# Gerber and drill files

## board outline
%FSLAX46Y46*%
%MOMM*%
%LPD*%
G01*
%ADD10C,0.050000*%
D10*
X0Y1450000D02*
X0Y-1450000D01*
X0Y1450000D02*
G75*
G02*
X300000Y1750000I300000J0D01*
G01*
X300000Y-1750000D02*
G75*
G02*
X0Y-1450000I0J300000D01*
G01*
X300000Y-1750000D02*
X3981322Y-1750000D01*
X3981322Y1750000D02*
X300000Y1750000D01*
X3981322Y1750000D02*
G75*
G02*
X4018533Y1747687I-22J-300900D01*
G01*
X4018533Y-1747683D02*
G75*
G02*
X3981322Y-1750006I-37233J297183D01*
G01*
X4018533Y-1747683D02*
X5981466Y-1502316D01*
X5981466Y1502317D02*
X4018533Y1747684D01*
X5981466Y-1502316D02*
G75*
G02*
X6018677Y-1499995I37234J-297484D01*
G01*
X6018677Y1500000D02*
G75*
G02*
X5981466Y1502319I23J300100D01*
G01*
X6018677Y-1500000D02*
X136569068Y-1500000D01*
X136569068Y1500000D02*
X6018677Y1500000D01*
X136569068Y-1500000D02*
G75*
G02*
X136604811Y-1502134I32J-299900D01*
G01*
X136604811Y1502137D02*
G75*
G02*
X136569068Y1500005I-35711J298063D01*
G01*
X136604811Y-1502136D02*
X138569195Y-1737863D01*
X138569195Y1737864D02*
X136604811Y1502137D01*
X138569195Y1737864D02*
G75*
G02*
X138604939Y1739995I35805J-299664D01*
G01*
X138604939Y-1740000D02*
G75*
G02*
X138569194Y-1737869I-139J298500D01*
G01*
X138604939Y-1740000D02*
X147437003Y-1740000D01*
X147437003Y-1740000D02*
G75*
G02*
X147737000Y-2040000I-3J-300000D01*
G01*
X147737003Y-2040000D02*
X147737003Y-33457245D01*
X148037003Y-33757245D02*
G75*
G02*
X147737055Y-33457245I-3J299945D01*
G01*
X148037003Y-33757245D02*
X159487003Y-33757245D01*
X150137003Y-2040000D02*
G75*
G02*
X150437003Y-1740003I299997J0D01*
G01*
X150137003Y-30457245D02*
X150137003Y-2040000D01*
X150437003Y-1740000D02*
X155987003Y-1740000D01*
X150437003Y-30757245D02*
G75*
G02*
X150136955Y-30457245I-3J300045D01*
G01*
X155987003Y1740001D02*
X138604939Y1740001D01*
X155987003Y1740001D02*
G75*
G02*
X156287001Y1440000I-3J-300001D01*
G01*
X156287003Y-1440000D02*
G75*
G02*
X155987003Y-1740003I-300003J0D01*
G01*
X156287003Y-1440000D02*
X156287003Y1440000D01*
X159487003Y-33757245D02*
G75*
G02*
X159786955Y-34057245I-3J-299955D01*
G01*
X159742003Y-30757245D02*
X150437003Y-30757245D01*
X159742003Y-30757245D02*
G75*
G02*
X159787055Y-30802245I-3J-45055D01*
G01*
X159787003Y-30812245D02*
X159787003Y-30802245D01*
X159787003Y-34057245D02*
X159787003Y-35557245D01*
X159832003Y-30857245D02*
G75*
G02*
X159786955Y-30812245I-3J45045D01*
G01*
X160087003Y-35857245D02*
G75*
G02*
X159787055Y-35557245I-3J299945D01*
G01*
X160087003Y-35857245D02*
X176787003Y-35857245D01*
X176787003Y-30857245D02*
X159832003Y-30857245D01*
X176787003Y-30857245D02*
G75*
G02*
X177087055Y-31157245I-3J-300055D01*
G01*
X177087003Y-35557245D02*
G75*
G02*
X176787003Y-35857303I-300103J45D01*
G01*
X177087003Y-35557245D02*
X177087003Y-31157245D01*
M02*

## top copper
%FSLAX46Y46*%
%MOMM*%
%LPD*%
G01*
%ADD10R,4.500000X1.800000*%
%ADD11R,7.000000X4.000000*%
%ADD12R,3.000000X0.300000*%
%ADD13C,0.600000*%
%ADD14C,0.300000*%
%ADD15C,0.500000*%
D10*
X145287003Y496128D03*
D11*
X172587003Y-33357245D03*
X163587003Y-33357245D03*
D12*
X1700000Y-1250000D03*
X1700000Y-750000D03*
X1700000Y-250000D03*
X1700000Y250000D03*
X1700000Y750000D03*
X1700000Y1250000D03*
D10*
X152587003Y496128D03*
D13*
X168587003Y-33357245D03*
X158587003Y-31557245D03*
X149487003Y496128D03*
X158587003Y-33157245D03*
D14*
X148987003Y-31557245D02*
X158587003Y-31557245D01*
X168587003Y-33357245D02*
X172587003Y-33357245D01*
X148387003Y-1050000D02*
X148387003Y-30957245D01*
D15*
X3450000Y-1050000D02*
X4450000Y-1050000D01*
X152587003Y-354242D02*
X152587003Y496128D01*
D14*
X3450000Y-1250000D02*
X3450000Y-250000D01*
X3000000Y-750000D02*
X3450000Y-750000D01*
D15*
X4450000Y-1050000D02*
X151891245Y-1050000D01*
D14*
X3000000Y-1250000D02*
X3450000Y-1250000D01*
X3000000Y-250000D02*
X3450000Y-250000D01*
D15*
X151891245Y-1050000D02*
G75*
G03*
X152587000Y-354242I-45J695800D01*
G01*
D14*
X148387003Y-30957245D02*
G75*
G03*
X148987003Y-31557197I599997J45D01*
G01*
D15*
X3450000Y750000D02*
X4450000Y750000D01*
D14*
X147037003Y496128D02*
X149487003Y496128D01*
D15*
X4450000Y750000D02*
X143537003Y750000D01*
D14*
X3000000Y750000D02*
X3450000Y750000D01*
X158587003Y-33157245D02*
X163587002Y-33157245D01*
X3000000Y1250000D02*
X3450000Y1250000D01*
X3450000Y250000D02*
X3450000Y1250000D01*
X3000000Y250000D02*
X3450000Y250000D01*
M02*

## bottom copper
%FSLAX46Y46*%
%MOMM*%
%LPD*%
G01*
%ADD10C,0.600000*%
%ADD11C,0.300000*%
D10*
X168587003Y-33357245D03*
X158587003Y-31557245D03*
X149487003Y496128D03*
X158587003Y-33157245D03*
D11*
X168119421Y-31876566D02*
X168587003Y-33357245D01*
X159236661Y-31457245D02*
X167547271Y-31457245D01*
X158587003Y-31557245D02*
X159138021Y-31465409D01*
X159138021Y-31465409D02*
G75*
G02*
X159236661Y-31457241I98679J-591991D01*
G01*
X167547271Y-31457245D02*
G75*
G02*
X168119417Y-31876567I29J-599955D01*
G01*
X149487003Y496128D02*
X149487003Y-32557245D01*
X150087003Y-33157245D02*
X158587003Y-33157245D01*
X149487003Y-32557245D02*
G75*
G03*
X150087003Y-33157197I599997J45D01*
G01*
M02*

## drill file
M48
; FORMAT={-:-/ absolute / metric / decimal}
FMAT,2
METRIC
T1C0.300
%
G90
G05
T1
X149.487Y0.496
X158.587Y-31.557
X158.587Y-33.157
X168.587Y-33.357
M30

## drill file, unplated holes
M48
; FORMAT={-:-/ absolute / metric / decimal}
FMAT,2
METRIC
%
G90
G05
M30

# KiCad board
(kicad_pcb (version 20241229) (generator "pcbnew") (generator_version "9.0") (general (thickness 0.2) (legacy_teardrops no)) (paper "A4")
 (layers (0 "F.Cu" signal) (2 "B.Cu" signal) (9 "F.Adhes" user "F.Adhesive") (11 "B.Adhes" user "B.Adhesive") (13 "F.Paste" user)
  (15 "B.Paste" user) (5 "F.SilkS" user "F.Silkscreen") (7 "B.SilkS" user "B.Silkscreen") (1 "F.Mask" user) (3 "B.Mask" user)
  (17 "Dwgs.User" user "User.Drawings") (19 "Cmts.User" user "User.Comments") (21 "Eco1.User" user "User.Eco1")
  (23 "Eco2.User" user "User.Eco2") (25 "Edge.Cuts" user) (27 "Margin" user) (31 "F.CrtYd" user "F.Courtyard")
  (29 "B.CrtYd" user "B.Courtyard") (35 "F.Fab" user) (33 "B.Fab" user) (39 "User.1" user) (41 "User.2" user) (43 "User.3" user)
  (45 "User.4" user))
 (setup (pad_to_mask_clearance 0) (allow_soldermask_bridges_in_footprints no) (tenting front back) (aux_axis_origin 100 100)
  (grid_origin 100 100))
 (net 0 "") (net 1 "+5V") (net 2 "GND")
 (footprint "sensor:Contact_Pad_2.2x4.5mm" (layer "F.Cu") (at 245.287003 99.503872)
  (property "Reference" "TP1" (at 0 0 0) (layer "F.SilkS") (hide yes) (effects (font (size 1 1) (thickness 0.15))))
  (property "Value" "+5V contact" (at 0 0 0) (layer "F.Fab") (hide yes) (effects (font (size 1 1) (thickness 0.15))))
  (pad "1" smd rect (at 0 0) (size 4.5 1.8) (layers "F.Cu" "F.Mask") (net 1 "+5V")))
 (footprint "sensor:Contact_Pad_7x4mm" (layer "F.Cu") (at 272.587003 133.357245)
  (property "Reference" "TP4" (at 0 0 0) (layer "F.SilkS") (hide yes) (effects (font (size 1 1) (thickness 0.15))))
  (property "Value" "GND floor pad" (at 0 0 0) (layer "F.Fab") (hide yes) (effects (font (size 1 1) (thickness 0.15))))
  (pad "1" smd rect (at 0 0) (size 7 4) (layers "F.Cu" "F.Mask") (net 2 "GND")))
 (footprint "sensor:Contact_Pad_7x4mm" (layer "F.Cu") (at 263.587003 133.357245)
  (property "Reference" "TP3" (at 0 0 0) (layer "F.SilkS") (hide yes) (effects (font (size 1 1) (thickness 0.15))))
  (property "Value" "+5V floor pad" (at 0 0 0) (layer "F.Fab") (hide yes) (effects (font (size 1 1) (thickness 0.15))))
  (pad "1" smd rect (at 0 0) (size 7 4) (layers "F.Cu" "F.Mask") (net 1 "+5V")))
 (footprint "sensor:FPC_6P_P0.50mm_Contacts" (layer "F.Cu") (at 101.7 100)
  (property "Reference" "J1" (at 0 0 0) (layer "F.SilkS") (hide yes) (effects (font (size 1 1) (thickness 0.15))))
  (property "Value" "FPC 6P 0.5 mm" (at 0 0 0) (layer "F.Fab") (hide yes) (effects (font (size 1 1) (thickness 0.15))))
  (pad "1" smd rect (at 0 1.25) (size 3 0.3) (layers "F.Cu" "F.Mask") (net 2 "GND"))
  (pad "2" smd rect (at 0 0.75) (size 3 0.3) (layers "F.Cu" "F.Mask") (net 2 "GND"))
  (pad "3" smd rect (at 0 0.25) (size 3 0.3) (layers "F.Cu" "F.Mask") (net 2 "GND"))
  (pad "4" smd rect (at 0 -0.25) (size 3 0.3) (layers "F.Cu" "F.Mask") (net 1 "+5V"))
  (pad "5" smd rect (at 0 -0.75) (size 3 0.3) (layers "F.Cu" "F.Mask") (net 1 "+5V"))
  (pad "6" smd rect (at 0 -1.25) (size 3 0.3) (layers "F.Cu" "F.Mask") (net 1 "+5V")))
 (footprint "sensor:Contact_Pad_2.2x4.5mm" (layer "F.Cu") (at 252.587003 99.503872)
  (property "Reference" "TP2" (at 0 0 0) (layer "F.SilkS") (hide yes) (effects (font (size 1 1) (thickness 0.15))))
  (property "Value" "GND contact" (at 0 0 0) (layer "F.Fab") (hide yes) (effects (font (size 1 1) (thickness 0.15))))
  (pad "1" smd rect (at 0 0) (size 4.5 1.8) (layers "F.Cu" "F.Mask") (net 2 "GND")))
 (gr_line (start 100 98.55) (end 100 101.45) (stroke (width 0.05) (type default)) (layer "Edge.Cuts"))
 (gr_arc (start 100 98.55) (mid 100.087868 98.337868) (end 100.3 98.25) (stroke (width 0.05) (type default)) (layer "Edge.Cuts"))
 (gr_arc (start 100.3 101.75) (mid 100.087868 101.662132) (end 100 101.45) (stroke (width 0.05) (type default)) (layer "Edge.Cuts"))
 (gr_line (start 100.3 101.75) (end 103.981322 101.75) (stroke (width 0.05) (type default)) (layer "Edge.Cuts"))
 (gr_line (start 103.981322 98.25) (end 100.3 98.25) (stroke (width 0.05) (type default)) (layer "Edge.Cuts"))
 (gr_arc (start 103.981322 98.25) (mid 103.999963 98.250581) (end 104.018533 98.252316) (stroke (width 0.05) (type default))
  (layer "Edge.Cuts"))
 (gr_arc (start 104.018533 101.747683) (mid 103.999964 101.749421) (end 103.981322 101.75) (stroke (width 0.05) (type default))
  (layer "Edge.Cuts"))
 (gr_line (start 104.018533 101.747683) (end 105.981466 101.502316) (stroke (width 0.05) (type default)) (layer "Edge.Cuts"))
 (gr_line (start 105.981466 98.497683) (end 104.018533 98.252316) (stroke (width 0.05) (type default)) (layer "Edge.Cuts"))
 (gr_arc (start 105.981466 101.502316) (mid 106.000036 101.500579) (end 106.018677 101.5) (stroke (width 0.05) (type default))
  (layer "Edge.Cuts"))
 (gr_arc (start 106.018677 98.5) (mid 106.000036 98.49942) (end 105.981466 98.497683) (stroke (width 0.05) (type default))
  (layer "Edge.Cuts"))
 (gr_line (start 106.018677 101.5) (end 236.569068 101.5) (stroke (width 0.05) (type default)) (layer "Edge.Cuts"))
 (gr_line (start 236.569068 98.5) (end 106.018677 98.5) (stroke (width 0.05) (type default)) (layer "Edge.Cuts"))
 (gr_arc (start 236.569068 101.5) (mid 236.586971 101.500534) (end 236.604811 101.502136) (stroke (width 0.05) (type default))
  (layer "Edge.Cuts"))
 (gr_arc (start 236.604811 98.497863) (mid 236.586971 98.499465) (end 236.569068 98.5) (stroke (width 0.05) (type default))
  (layer "Edge.Cuts"))
 (gr_line (start 236.604811 101.502136) (end 238.569195 101.737863) (stroke (width 0.05) (type default)) (layer "Edge.Cuts"))
 (gr_line (start 238.569195 98.262136) (end 236.604811 98.497863) (stroke (width 0.05) (type default)) (layer "Edge.Cuts"))
 (gr_arc (start 238.569195 98.262136) (mid 238.587035 98.260537) (end 238.604939 98.259999) (stroke (width 0.05) (type default))
  (layer "Edge.Cuts"))
 (gr_arc (start 238.604939 101.74) (mid 238.587035 101.739468) (end 238.569195 101.737863) (stroke (width 0.05) (type default))
  (layer "Edge.Cuts"))
 (gr_line (start 238.604939 101.74) (end 247.437003 101.74) (stroke (width 0.05) (type default)) (layer "Edge.Cuts"))
 (gr_arc (start 247.437003 101.74) (mid 247.649135 101.827867) (end 247.737003 102.04) (stroke (width 0.05) (type default))
  (layer "Edge.Cuts"))
 (gr_line (start 247.737003 102.04) (end 247.737003 133.457245) (stroke (width 0.05) (type default)) (layer "Edge.Cuts"))
 (gr_arc (start 248.037003 133.757245) (mid 247.824853 133.669381) (end 247.737003 133.457245) (stroke (width 0.05) (type default))
  (layer "Edge.Cuts"))
 (gr_line (start 248.037003 133.757245) (end 259.487003 133.757245) (stroke (width 0.05) (type default)) (layer "Edge.Cuts"))
 (gr_arc (start 250.137003 102.04) (mid 250.224871 101.827867) (end 250.437003 101.74) (stroke (width 0.05) (type default))
  (layer "Edge.Cuts"))
 (gr_line (start 250.137003 130.457245) (end 250.137003 102.04) (stroke (width 0.05) (type default)) (layer "Edge.Cuts"))
 (gr_line (start 250.437003 101.74) (end 255.987003 101.74) (stroke (width 0.05) (type default)) (layer "Edge.Cuts"))
 (gr_arc (start 250.437003 130.757245) (mid 250.224871 130.669377) (end 250.137003 130.457245) (stroke (width 0.05) (type default))
  (layer "Edge.Cuts"))
 (gr_line (start 255.987003 98.259999) (end 238.604939 98.259999) (stroke (width 0.05) (type default)) (layer "Edge.Cuts"))
 (gr_arc (start 255.987003 98.259999) (mid 256.199134 98.347868) (end 256.287003 98.56) (stroke (width 0.05) (type default))
  (layer "Edge.Cuts"))
 (gr_arc (start 256.287003 101.44) (mid 256.199135 101.652133) (end 255.987003 101.74) (stroke (width 0.05) (type default))
  (layer "Edge.Cuts"))
 (gr_line (start 256.287003 101.44) (end 256.287003 98.56) (stroke (width 0.05) (type default)) (layer "Edge.Cuts"))
 (gr_arc (start 259.487003 133.757245) (mid 259.699135 133.845113) (end 259.787003 134.057245) (stroke (width 0.05) (type default))
  (layer "Edge.Cuts"))
 (gr_line (start 259.742003 130.757245) (end 250.437003 130.757245) (stroke (width 0.05) (type default)) (layer "Edge.Cuts"))
 (gr_arc (start 259.742003 130.757245) (mid 259.773805 130.770429) (end 259.787003 130.802245) (stroke (width 0.05) (type default))
  (layer "Edge.Cuts"))
 (gr_line (start 259.787003 130.812245) (end 259.787003 130.802245) (stroke (width 0.05) (type default)) (layer "Edge.Cuts"))
 (gr_line (start 259.787003 134.057245) (end 259.787003 135.557245) (stroke (width 0.05) (type default)) (layer "Edge.Cuts"))
 (gr_arc (start 259.832003 130.857245) (mid 259.800184 130.844065) (end 259.787003 130.812245) (stroke (width 0.05) (type default))
  (layer "Edge.Cuts"))
 (gr_arc (start 260.087003 135.857245) (mid 259.874853 135.769381) (end 259.787003 135.557245) (stroke (width 0.05) (type default))
  (layer "Edge.Cuts"))
 (gr_line (start 260.087003 135.857245) (end 276.787003 135.857245) (stroke (width 0.05) (type default)) (layer "Edge.Cuts"))
 (gr_line (start 276.787003 130.857245) (end 259.832003 130.857245) (stroke (width 0.05) (type default)) (layer "Edge.Cuts"))
 (gr_arc (start 276.787003 130.857245) (mid 276.999117 130.945117) (end 277.087003 131.157245) (stroke (width 0.05) (type default))
  (layer "Edge.Cuts"))
 (gr_arc (start 277.087003 135.557245) (mid 276.999119 135.769349) (end 276.787003 135.857245) (stroke (width 0.05) (type default))
  (layer "Edge.Cuts"))
 (gr_line (start 277.087003 135.557245) (end 277.087003 131.157245) (stroke (width 0.05) (type default)) (layer "Edge.Cuts"))
 (segment (start 248.987003 131.557245) (end 258.587003 131.557245) (width 0.3) (layer "F.Cu") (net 2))
 (segment (start 268.587003 133.357245) (end 272.587003 133.357245) (width 0.3) (layer "F.Cu") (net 2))
 (segment (start 248.387003 101.05) (end 248.387003 130.957245) (width 0.3) (layer "F.Cu") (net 2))
 (segment (start 103.45 101.05) (end 104.45 101.05) (width 0.5) (layer "F.Cu") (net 2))
 (segment (start 252.587003 100.354242) (end 252.587003 99.503872) (width 0.5) (layer "F.Cu") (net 2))
 (segment (start 103.45 101.25) (end 103.45 100.25) (width 0.3) (layer "F.Cu") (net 2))
 (segment (start 103 100.75) (end 103.45 100.75) (width 0.3) (layer "F.Cu") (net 2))
 (segment (start 104.45 101.05) (end 251.891245 101.05) (width 0.5) (layer "F.Cu") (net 2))
 (segment (start 103 101.25) (end 103.45 101.25) (width 0.3) (layer "F.Cu") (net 2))
 (segment (start 103 100.25) (end 103.45 100.25) (width 0.3) (layer "F.Cu") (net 2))
 (via (at 268.587003 133.357245) (size 0.6) (drill 0.3) (layers "F.Cu" "B.Cu") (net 2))
 (via (at 258.587003 131.557245) (size 0.6) (drill 0.3) (layers "F.Cu" "B.Cu") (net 2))
 (arc (start 251.891245 101.05) (mid 252.38322 100.846217) (end 252.587003 100.354242) (width 0.5) (layer "F.Cu") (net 2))
 (arc (start 248.387003 130.957245) (mid 248.562739 131.381509) (end 248.987003 131.557245) (width 0.3) (layer "F.Cu") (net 2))
 (segment (start 268.119421 131.876566) (end 268.587003 133.357245) (width 0.3) (layer "B.Cu") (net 2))
 (segment (start 259.236661 131.457245) (end 267.547271 131.457245) (width 0.3) (layer "B.Cu") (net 2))
 (segment (start 258.587003 131.557245) (end 259.138021 131.465409) (width 0.3) (layer "B.Cu") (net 2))
 (arc (start 259.138021 131.465409) (mid 259.187173 131.45929) (end 259.236661 131.457245) (width 0.3) (layer "B.Cu") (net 2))
 (arc (start 267.547271 131.457245) (mid 267.901949 131.573299) (end 268.119421 131.876566) (width 0.3) (layer "B.Cu") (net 2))
 (segment (start 103.45 99.25) (end 104.45 99.25) (width 0.5) (layer "F.Cu") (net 1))
 (segment (start 247.037003 99.503872) (end 249.487003 99.503872) (width 0.3) (layer "F.Cu") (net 1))
 (segment (start 104.45 99.25) (end 243.537003 99.25) (width 0.5) (layer "F.Cu") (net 1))
 (segment (start 103 99.25) (end 103.45 99.25) (width 0.3) (layer "F.Cu") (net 1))
 (segment (start 258.587003 133.157245) (end 263.587002 133.157245) (width 0.3) (layer "F.Cu") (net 1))
 (segment (start 103 98.75) (end 103.45 98.75) (width 0.3) (layer "F.Cu") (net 1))
 (segment (start 103.45 99.75) (end 103.45 98.75) (width 0.3) (layer "F.Cu") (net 1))
 (segment (start 103 99.75) (end 103.45 99.75) (width 0.3) (layer "F.Cu") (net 1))
 (via (at 249.487003 99.503872) (size 0.6) (drill 0.3) (layers "F.Cu" "B.Cu") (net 1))
 (via (at 258.587003 133.157245) (size 0.6) (drill 0.3) (layers "F.Cu" "B.Cu") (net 1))
 (segment (start 249.487003 99.503872) (end 249.487003 132.557245) (width 0.3) (layer "B.Cu") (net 1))
 (segment (start 250.087003 133.157245) (end 258.587003 133.157245) (width 0.3) (layer "B.Cu") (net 1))
 (arc (start 249.487003 132.557245) (mid 249.662739 132.981509) (end 250.087003 133.157245) (width 0.3) (layer "B.Cu") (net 1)))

